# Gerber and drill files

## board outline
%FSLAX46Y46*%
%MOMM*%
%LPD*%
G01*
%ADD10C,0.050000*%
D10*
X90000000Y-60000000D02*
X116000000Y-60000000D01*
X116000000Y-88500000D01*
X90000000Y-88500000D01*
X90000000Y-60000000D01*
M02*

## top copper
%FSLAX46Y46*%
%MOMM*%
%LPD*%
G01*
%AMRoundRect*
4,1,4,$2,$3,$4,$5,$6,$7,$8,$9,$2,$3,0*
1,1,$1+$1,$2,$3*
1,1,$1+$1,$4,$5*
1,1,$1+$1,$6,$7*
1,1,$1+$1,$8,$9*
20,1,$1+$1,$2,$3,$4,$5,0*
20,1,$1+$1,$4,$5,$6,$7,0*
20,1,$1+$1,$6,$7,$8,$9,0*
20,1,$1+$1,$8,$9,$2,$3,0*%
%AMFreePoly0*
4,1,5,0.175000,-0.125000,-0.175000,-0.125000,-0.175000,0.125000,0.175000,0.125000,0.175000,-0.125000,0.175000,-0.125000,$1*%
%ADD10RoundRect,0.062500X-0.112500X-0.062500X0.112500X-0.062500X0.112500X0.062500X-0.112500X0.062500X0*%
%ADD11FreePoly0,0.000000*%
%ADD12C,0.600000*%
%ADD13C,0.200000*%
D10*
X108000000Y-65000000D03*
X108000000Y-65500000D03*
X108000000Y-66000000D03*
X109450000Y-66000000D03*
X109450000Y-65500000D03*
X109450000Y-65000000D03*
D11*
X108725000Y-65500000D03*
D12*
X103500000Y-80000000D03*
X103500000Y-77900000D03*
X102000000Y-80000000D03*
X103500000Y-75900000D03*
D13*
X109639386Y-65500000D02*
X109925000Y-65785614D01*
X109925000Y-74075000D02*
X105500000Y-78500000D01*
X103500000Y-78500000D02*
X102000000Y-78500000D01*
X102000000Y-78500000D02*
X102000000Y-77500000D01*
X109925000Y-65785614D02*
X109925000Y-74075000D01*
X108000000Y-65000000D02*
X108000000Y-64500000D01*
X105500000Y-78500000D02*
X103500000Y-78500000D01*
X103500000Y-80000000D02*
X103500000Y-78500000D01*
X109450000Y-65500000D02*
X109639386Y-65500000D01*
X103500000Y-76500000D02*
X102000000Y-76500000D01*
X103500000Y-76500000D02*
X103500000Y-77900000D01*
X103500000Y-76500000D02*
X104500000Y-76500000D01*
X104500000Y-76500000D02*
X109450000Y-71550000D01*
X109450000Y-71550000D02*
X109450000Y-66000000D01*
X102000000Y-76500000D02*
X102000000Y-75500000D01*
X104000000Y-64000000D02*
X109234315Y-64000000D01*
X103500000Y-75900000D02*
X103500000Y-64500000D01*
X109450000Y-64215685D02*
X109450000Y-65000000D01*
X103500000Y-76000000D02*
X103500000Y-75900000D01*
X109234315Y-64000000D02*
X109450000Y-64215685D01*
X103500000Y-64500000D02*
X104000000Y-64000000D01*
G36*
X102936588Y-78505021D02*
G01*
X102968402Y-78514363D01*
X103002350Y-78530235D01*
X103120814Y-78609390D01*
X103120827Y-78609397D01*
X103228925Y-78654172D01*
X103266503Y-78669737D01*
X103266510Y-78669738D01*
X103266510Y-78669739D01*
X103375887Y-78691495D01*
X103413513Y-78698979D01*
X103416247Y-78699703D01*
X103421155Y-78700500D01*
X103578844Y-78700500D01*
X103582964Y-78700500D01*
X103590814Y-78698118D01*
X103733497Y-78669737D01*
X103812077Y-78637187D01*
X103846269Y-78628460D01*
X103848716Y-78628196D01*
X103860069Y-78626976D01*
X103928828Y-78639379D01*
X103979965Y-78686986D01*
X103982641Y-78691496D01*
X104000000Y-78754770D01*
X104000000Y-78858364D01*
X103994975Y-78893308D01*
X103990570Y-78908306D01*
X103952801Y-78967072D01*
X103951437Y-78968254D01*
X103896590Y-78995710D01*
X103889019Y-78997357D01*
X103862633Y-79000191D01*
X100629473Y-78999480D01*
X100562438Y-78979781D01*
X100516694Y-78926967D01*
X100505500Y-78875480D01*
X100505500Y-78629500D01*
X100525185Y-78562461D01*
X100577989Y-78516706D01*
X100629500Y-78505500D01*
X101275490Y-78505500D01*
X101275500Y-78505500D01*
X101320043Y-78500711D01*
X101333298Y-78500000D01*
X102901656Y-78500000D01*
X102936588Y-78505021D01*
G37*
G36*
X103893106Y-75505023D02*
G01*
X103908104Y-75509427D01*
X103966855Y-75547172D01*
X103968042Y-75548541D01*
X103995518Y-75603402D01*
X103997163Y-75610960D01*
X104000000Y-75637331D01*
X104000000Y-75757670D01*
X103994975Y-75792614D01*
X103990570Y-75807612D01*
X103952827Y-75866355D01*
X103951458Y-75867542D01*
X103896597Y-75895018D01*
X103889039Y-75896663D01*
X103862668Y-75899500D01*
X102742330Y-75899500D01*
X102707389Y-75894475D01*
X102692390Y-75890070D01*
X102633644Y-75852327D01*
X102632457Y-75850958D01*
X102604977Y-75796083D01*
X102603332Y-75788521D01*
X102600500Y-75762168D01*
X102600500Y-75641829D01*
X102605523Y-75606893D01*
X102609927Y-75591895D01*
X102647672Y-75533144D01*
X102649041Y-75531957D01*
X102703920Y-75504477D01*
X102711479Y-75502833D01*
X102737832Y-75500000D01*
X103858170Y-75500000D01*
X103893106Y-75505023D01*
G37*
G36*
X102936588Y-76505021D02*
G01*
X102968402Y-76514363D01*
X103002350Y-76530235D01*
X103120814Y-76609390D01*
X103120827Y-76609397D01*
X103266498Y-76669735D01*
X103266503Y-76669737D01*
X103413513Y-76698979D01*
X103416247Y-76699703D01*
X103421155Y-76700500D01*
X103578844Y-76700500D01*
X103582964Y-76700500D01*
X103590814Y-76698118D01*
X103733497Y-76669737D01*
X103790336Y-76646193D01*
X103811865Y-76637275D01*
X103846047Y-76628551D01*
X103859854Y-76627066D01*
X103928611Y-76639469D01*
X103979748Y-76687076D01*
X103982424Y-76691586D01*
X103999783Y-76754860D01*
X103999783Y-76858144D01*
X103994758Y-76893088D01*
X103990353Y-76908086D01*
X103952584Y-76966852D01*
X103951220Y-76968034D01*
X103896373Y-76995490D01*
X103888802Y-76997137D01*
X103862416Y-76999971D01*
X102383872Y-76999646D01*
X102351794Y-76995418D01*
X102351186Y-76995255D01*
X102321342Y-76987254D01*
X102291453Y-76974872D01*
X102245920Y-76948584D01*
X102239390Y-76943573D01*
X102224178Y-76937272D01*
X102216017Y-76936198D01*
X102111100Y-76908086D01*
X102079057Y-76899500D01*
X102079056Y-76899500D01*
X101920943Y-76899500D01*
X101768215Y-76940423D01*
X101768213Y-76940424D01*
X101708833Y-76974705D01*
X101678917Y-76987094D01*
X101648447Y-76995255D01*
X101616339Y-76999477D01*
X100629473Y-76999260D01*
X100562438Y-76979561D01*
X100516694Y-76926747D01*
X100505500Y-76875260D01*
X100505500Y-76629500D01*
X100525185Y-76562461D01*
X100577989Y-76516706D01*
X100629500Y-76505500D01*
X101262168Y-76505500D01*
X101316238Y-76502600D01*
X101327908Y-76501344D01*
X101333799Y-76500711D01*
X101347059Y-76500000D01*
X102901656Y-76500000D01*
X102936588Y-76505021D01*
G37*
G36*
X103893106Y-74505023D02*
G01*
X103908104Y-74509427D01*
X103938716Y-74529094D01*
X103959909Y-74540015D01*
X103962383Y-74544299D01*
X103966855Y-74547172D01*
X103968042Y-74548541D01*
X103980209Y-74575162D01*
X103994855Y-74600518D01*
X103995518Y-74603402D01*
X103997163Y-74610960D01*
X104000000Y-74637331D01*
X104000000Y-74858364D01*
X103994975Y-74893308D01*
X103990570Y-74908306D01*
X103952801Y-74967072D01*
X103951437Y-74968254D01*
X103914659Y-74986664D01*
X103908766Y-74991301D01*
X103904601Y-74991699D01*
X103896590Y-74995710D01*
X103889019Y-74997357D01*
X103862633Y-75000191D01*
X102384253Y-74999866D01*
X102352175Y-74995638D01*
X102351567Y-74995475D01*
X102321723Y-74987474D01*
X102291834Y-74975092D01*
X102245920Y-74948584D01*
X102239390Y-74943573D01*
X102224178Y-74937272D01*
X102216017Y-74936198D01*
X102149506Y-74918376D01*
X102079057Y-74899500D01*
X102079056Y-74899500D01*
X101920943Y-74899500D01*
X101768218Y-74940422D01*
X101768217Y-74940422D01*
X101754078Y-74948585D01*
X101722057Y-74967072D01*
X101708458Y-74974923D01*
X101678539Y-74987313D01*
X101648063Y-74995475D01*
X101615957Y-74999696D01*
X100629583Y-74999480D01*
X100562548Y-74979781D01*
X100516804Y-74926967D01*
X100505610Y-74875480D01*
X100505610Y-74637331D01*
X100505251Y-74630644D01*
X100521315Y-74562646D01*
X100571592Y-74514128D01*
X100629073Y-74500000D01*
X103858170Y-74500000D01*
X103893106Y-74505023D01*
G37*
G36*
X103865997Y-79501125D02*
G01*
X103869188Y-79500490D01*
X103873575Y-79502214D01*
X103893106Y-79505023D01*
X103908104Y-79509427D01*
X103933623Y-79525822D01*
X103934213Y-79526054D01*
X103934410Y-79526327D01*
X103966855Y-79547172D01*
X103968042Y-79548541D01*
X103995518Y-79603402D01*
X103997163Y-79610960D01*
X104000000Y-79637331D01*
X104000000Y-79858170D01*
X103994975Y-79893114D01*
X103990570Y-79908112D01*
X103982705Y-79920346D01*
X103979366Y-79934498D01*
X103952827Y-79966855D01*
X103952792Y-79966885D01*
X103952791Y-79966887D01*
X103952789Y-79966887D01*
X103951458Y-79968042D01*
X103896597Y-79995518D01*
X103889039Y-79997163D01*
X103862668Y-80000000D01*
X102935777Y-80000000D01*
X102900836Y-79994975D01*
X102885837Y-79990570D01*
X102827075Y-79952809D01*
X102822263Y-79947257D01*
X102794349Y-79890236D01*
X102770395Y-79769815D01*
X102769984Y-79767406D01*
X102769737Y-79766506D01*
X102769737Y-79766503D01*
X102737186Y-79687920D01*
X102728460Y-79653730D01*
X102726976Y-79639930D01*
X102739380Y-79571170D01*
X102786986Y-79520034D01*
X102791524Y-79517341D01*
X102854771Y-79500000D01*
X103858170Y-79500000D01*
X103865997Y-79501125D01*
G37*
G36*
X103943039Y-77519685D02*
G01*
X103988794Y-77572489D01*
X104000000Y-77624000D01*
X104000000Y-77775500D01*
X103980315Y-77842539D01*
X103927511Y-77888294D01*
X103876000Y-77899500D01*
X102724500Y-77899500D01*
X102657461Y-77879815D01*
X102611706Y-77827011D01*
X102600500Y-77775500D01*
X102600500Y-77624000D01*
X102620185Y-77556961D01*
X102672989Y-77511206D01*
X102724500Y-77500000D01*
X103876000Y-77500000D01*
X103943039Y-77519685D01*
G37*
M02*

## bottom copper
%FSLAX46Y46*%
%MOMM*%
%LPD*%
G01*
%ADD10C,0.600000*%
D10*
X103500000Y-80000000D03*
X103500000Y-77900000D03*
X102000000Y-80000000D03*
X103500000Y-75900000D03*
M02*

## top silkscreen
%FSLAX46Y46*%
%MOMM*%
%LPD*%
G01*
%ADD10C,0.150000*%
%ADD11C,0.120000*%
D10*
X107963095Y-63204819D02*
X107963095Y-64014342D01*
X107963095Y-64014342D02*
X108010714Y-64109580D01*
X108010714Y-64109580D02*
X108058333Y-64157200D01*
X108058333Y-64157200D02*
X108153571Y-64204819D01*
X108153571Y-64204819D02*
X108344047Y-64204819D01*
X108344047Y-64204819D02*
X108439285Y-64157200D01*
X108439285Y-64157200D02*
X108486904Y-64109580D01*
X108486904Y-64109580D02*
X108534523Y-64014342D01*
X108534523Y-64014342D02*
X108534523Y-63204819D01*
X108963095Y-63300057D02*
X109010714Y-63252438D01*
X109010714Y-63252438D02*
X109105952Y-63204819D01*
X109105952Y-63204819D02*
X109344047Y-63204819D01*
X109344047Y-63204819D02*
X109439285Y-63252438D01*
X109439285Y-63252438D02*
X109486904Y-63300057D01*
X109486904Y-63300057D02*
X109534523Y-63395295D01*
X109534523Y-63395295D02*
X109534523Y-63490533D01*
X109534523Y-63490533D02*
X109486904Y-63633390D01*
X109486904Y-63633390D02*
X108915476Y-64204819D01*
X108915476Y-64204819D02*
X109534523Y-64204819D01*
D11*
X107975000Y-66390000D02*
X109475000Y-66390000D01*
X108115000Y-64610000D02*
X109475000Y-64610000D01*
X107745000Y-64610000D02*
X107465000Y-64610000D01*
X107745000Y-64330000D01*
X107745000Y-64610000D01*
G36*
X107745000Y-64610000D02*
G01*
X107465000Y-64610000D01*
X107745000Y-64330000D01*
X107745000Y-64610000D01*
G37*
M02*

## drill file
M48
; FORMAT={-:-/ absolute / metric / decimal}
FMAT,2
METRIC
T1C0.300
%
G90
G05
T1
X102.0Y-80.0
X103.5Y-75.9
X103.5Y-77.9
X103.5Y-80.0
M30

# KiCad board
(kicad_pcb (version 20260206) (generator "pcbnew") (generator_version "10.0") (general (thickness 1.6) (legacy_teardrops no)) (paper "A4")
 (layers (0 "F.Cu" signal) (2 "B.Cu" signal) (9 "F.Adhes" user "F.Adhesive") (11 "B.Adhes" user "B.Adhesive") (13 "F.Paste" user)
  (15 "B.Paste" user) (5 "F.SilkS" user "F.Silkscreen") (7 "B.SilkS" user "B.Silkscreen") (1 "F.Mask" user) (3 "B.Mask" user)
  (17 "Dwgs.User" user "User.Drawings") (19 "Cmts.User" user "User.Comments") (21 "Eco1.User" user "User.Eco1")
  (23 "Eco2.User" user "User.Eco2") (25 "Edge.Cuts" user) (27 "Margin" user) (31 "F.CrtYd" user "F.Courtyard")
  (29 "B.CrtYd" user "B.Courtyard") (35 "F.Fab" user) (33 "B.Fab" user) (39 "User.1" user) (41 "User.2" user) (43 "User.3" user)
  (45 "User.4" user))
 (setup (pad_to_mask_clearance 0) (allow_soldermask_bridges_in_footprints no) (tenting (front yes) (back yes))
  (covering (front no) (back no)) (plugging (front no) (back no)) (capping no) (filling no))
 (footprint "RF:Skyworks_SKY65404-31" (layer "F.Cu") (at 108.725 65.5)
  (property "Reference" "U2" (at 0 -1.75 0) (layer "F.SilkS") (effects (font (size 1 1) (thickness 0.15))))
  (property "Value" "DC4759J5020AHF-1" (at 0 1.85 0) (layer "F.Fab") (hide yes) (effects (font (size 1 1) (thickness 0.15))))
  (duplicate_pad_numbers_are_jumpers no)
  (fp_line (start -0.75 0.89) (end 0.75 0.89) (stroke (width 0.12) (type solid)) (layer "F.SilkS"))
  (fp_line (start -0.61 -0.89) (end 0.75 -0.89) (stroke (width 0.12) (type solid)) (layer "F.SilkS"))
  (fp_poly
   (pts (xy -0.98 -0.89) (xy -1.26 -0.89) (xy -0.98 -1.17) (xy -0.98 -0.89)) (stroke (width 0.12) (type solid)) (fill yes) (layer "F.SilkS"))
  (pad "1" smd roundrect (at -0.725 -0.5) (size 0.35 0.25) (layers "F.Cu" "F.Mask" "F.Paste") (roundrect_rratio 0.25)
   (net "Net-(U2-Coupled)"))
  (pad "2" smd roundrect (at -0.725 0) (size 0.35 0.25) (layers "F.Cu" "F.Mask" "F.Paste") (roundrect_rratio 0.25) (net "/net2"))
  (pad "3" smd roundrect (at -0.725 0.5) (size 0.35 0.25) (layers "F.Cu" "F.Mask" "F.Paste") (roundrect_rratio 0.25) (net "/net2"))
  (pad "4" smd roundrect (at 0.725 0.5) (size 0.35 0.25) (layers "F.Cu" "F.Mask" "F.Paste") (roundrect_rratio 0.25) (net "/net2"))
  (pad "5" smd roundrect (at 0.725 0) (size 0.35 0.25) (layers "F.Cu" "F.Mask" "F.Paste") (roundrect_rratio 0.25) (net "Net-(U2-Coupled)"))
  (pad "6" smd roundrect (at 0.725 -0.5) (size 0.35 0.25) (layers "F.Cu" "F.Mask" "F.Paste") (roundrect_rratio 0.25) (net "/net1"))
  (pad "7" smd custom (at 0 0) (size 0.35 0.25) (layers "F.Cu" "F.Mask" "F.Paste") (zone_connect 0)
   (options (clearance outline) (anchor rect)) (primitives)))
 (gr_rect (start 90 60) (end 116 88.5) (stroke (width 0.05) (type default)) (fill no) (layer "Edge.Cuts"))
 (segment (start 109.639386 65.5) (end 109.925 65.785614) (width 0.2) (layer "F.Cu") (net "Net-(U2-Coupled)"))
 (segment (start 109.925 74.075) (end 105.5 78.5) (width 0.2) (layer "F.Cu") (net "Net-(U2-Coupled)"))
 (segment (start 103.5 78.5) (end 102 78.5) (width 0.2) (layer "F.Cu") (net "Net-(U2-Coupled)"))
 (segment (start 102 78.5) (end 102 77.5) (width 0.2) (layer "F.Cu") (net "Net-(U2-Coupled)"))
 (segment (start 109.925 65.785614) (end 109.925 74.075) (width 0.2) (layer "F.Cu") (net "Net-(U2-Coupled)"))
 (segment (start 108 65) (end 108 64.5) (width 0.2) (layer "F.Cu") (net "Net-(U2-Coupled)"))
 (segment (start 105.5 78.5) (end 103.5 78.5) (width 0.2) (layer "F.Cu") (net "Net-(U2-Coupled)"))
 (segment (start 103.5 80) (end 103.5 78.5) (width 0.2) (layer "F.Cu") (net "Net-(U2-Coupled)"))
 (segment (start 109.45 65.5) (end 109.639386 65.5) (width 0.2) (layer "F.Cu") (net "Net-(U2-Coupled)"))
 (via (at 103.5 80) (size 0.6) (drill 0.3) (layers "F.Cu" "B.Cu") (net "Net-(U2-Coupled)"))
 (segment (start 103.5 76.5) (end 102 76.5) (width 0.2) (layer "F.Cu") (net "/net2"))
 (segment (start 103.5 76.5) (end 103.5 77.9) (width 0.2) (layer "F.Cu") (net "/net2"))
 (segment (start 103.5 76.5) (end 104.5 76.5) (width 0.2) (layer "F.Cu") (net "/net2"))
 (segment (start 104.5 76.5) (end 109.45 71.55) (width 0.2) (layer "F.Cu") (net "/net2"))
 (segment (start 109.45 71.55) (end 109.45 66) (width 0.2) (layer "F.Cu") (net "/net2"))
 (segment (start 102 76.5) (end 102 75.5) (width 0.2) (layer "F.Cu") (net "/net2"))
 (via (at 103.5 77.9) (size 0.6) (drill 0.3) (layers "F.Cu" "B.Cu") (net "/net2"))
 (segment (start 104 64) (end 109.234315 64) (width 0.2) (layer "F.Cu") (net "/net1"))
 (segment (start 103.5 75.9) (end 103.5 64.5) (width 0.2) (layer "F.Cu") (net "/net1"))
 (segment (start 109.45 64.215685) (end 109.45 65) (width 0.2) (layer "F.Cu") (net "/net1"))
 (segment (start 103.5 76) (end 103.5 75.9) (width 0.2) (layer "F.Cu") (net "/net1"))
 (segment (start 109.234315 64) (end 109.45 64.215685) (width 0.2) (layer "F.Cu") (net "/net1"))
 (segment (start 103.5 64.5) (end 104 64) (width 0.2) (layer "F.Cu") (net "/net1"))
 (via (at 102 80) (size 0.6) (drill 0.3) (layers "F.Cu" "B.Cu") (free yes) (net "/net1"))
 (via (at 103.5 75.9) (size 0.6) (drill 0.3) (layers "F.Cu" "B.Cu") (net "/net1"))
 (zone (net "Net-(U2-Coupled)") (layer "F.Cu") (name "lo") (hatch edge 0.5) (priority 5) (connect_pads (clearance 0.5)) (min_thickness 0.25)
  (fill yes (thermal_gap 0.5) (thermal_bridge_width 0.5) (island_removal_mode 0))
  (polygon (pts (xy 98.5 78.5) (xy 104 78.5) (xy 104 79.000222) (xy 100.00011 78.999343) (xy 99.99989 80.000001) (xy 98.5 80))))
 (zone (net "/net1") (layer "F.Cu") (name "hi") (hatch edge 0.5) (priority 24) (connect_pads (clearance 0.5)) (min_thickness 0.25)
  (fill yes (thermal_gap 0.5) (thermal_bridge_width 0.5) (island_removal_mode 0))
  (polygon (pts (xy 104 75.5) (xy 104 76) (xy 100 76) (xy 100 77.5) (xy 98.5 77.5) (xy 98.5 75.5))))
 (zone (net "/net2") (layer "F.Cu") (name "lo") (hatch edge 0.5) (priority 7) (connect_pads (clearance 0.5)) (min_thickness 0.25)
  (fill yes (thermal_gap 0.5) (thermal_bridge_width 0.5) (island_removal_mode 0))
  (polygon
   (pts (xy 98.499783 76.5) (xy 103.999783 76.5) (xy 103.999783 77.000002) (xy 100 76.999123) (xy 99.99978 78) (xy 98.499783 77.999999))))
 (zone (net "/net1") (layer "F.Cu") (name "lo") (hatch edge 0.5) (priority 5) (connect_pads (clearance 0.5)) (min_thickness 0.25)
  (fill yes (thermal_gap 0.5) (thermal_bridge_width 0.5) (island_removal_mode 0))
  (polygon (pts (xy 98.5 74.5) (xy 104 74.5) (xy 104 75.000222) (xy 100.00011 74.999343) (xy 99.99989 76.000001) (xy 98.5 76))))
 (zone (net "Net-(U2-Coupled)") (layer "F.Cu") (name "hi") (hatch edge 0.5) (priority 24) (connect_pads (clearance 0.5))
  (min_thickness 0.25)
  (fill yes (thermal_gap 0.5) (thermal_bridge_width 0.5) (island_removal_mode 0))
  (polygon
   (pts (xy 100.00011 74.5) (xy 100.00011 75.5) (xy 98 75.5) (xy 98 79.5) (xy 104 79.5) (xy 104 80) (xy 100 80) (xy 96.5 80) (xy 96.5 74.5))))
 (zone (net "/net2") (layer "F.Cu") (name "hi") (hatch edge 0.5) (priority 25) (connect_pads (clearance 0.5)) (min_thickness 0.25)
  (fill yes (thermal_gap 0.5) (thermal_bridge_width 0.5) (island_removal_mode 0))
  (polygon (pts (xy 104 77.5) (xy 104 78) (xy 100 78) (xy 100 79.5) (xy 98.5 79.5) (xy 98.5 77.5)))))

